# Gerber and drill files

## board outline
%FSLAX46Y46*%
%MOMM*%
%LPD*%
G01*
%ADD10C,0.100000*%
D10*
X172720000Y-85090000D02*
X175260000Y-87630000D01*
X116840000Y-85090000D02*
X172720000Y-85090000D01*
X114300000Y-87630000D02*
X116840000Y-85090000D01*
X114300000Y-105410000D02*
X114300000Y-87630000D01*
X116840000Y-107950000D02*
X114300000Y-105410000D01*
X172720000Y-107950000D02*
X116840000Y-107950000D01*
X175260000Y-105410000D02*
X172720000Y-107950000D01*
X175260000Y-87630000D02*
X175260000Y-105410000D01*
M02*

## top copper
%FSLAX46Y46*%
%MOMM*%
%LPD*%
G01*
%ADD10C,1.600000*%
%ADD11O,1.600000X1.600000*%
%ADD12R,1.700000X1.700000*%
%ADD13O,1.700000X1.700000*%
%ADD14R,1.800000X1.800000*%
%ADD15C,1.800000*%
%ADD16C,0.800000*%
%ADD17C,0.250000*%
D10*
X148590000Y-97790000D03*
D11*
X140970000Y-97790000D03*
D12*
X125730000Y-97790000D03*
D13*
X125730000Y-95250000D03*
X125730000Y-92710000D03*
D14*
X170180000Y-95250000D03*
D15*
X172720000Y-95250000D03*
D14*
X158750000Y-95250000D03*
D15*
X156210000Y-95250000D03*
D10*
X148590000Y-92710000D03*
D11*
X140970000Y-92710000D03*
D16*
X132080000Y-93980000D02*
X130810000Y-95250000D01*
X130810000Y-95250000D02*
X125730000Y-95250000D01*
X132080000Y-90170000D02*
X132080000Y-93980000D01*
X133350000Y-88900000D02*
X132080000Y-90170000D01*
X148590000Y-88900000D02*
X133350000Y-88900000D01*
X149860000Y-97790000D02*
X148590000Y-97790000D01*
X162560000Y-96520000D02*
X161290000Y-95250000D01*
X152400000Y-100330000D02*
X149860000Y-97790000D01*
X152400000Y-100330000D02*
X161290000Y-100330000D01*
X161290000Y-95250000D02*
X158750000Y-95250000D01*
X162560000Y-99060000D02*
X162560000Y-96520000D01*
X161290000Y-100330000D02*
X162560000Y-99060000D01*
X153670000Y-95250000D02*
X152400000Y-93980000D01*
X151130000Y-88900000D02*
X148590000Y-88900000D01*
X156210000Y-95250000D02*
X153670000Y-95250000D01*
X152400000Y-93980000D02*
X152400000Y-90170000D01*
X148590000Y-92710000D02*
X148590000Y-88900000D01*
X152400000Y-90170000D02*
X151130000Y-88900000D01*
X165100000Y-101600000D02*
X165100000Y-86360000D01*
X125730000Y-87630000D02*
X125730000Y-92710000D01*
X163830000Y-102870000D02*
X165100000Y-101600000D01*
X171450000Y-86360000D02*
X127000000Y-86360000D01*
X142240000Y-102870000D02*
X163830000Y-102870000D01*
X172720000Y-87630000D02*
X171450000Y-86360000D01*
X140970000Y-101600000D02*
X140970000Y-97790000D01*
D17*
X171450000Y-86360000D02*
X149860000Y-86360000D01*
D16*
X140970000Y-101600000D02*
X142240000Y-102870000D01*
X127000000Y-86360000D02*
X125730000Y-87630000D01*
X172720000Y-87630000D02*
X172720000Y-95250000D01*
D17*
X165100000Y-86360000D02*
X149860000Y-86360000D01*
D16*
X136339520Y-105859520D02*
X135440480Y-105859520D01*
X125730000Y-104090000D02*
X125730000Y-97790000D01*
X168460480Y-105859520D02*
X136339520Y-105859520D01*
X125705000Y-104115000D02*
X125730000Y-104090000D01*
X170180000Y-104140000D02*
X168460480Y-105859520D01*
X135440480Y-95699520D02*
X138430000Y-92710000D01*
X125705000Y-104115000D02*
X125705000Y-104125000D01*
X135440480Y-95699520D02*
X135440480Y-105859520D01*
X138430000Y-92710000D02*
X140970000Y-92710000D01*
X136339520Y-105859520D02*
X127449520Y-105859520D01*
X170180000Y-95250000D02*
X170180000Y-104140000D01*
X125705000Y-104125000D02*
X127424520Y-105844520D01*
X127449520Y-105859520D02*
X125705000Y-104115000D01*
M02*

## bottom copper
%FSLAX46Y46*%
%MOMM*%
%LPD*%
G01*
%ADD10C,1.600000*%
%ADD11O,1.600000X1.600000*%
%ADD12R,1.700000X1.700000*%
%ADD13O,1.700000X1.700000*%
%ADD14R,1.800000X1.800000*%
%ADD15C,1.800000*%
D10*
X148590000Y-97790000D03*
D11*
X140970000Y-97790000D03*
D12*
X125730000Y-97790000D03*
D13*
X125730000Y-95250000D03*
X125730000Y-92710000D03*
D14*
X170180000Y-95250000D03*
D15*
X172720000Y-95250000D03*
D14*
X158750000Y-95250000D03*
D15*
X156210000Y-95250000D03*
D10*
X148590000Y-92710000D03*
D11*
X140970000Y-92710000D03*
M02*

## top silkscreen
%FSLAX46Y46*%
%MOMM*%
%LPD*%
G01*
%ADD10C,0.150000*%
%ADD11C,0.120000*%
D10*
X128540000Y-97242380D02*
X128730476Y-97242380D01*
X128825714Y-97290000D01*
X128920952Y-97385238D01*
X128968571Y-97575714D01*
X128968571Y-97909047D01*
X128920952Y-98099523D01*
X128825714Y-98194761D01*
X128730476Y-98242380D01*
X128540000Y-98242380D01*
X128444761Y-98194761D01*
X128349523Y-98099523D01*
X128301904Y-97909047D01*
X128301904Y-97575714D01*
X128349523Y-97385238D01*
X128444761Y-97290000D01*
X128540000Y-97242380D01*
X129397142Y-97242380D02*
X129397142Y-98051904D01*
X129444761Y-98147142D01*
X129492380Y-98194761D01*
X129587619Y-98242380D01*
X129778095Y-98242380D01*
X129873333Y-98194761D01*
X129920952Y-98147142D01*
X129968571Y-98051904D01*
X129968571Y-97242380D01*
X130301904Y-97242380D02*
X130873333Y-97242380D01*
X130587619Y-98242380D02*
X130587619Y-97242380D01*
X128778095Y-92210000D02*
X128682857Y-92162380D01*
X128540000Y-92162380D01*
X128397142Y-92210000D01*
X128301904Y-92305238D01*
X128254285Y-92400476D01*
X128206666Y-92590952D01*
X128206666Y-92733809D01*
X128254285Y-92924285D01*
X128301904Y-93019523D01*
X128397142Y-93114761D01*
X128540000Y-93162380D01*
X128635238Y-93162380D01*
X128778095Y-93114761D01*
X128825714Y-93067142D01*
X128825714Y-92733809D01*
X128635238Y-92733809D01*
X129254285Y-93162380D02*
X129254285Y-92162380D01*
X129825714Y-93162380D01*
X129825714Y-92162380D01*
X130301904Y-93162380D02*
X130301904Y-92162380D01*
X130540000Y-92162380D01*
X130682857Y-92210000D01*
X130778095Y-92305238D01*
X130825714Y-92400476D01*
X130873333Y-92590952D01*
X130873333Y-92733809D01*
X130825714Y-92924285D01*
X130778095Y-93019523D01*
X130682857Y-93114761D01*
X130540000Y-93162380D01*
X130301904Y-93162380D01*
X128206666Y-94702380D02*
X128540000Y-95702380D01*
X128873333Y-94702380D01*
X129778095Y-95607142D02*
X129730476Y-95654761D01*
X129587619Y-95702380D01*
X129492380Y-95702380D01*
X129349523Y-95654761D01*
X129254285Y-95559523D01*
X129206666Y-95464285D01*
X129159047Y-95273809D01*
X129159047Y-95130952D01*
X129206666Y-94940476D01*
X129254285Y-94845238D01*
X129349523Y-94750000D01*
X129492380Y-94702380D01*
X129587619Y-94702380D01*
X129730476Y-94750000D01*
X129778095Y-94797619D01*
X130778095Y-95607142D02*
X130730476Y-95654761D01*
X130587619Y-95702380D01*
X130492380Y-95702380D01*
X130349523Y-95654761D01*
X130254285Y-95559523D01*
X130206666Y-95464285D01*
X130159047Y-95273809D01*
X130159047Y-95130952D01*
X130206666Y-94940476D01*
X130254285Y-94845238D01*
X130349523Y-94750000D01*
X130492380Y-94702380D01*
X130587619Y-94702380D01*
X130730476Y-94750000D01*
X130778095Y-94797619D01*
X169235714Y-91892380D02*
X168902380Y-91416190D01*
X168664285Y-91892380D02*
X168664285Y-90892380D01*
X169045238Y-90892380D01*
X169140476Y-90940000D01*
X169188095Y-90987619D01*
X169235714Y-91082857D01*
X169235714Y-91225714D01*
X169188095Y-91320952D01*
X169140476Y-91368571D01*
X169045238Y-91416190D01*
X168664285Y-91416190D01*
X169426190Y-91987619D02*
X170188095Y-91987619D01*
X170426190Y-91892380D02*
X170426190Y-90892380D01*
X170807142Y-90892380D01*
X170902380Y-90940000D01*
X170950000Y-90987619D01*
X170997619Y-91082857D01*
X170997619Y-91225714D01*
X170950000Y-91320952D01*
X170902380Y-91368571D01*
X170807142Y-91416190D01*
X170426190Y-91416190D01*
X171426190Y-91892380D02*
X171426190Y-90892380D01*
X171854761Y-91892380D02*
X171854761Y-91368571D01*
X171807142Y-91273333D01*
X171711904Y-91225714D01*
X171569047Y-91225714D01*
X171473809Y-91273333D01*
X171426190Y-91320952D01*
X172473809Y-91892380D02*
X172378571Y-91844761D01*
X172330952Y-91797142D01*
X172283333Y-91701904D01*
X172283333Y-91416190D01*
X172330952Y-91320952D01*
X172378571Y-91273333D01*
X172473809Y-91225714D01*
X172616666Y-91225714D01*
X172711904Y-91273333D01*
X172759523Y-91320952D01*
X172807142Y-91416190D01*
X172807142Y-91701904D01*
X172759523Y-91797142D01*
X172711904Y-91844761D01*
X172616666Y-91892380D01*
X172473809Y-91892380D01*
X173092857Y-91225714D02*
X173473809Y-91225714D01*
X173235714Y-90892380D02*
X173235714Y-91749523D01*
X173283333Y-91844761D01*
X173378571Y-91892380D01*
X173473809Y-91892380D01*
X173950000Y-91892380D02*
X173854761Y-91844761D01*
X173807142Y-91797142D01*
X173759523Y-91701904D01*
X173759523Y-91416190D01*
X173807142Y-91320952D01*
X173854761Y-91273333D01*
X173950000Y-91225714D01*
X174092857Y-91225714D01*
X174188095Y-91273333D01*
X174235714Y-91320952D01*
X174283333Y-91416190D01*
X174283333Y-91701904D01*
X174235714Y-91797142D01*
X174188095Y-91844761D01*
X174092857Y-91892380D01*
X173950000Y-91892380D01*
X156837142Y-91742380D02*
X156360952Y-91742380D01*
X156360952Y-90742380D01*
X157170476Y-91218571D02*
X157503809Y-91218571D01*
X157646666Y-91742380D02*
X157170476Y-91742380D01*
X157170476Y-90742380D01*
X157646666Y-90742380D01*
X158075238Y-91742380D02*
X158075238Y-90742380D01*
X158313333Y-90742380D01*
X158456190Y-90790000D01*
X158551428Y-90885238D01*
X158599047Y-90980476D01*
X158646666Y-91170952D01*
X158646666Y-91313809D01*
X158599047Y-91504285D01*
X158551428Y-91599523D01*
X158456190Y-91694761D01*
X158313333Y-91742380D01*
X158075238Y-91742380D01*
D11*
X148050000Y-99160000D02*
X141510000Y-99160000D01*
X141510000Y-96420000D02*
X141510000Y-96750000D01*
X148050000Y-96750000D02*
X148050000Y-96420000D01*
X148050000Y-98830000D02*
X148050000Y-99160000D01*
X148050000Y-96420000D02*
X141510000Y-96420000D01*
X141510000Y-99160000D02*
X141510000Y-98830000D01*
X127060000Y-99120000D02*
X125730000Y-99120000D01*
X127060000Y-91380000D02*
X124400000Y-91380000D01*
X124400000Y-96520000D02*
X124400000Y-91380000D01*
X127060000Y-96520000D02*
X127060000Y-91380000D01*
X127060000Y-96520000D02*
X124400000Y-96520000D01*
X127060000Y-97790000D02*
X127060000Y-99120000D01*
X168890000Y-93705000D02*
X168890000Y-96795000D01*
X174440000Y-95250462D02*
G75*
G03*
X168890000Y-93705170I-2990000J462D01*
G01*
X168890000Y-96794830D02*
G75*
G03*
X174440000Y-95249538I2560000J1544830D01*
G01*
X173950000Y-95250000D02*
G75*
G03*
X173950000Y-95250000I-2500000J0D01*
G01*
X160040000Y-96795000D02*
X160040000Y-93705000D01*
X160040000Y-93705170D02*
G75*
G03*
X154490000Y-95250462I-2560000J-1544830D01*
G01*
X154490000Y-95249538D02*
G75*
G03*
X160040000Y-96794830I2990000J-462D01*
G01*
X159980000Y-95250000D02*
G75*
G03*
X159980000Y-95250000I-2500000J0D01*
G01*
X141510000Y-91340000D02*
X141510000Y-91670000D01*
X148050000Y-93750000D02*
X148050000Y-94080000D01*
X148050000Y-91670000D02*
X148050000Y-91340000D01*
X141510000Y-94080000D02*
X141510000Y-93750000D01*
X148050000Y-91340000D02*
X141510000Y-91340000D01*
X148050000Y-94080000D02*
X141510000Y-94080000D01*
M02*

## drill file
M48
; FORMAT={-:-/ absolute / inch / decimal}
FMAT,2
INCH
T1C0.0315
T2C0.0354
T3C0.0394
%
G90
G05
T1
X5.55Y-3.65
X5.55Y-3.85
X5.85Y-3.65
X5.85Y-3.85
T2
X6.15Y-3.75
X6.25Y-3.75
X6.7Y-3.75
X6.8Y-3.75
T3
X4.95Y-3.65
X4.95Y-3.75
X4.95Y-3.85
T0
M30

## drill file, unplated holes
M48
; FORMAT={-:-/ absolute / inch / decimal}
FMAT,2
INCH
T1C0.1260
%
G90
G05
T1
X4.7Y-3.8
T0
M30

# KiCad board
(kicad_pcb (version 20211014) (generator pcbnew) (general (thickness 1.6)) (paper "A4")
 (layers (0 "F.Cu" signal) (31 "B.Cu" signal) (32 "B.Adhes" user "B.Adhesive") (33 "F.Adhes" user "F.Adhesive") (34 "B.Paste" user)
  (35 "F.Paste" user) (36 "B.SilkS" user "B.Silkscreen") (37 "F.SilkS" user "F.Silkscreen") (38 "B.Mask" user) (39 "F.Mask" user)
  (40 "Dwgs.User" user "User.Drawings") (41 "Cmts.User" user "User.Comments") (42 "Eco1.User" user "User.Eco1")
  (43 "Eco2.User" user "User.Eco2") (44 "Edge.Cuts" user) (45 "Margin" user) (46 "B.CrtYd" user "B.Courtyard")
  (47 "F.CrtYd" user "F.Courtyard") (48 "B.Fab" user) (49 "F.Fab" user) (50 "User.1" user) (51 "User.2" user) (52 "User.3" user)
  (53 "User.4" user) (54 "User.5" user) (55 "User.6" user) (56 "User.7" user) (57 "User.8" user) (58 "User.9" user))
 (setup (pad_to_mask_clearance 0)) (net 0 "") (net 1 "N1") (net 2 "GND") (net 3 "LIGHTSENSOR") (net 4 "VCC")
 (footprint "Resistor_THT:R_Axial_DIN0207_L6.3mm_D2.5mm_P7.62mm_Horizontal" (layer "F.Cu") (at 148.59 97.79 180)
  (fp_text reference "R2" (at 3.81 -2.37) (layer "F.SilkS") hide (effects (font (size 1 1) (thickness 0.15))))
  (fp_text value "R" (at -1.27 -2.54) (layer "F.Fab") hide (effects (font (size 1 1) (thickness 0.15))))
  (fp_line (start 0.54 -1.37) (end 7.08 -1.37) (layer "F.SilkS") (width 0.12))
  (fp_line (start 7.08 1.37) (end 7.08 1.04) (layer "F.SilkS") (width 0.12))
  (fp_line (start 0.54 1.04) (end 0.54 1.37) (layer "F.SilkS") (width 0.12))
  (fp_line (start 0.54 -1.04) (end 0.54 -1.37) (layer "F.SilkS") (width 0.12))
  (fp_line (start 0.54 1.37) (end 7.08 1.37) (layer "F.SilkS") (width 0.12))
  (fp_line (start 7.08 -1.37) (end 7.08 -1.04) (layer "F.SilkS") (width 0.12))
  (pad "1" thru_hole circle locked (at 0 0 180) (size 1.6 1.6) (drill 0.8) (layers *.Cu *.Mask) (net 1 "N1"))
  (pad "2" thru_hole oval locked (at 7.62 0 180) (size 1.6 1.6) (drill 0.8) (layers *.Cu *.Mask) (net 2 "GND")))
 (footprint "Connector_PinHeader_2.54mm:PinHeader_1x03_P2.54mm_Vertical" (layer "F.Cu") (at 125.73 97.79 180)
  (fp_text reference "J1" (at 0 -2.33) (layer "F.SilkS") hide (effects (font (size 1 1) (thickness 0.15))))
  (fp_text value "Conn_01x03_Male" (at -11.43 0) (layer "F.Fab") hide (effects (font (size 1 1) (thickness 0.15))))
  (fp_line (start -1.33 -1.33) (end 0 -1.33) (layer "F.SilkS") (width 0.12))
  (fp_line (start -1.33 6.41) (end 1.33 6.41) (layer "F.SilkS") (width 0.12))
  (fp_line (start 1.33 1.27) (end 1.33 6.41) (layer "F.SilkS") (width 0.12))
  (fp_line (start -1.33 1.27) (end -1.33 6.41) (layer "F.SilkS") (width 0.12))
  (fp_line (start -1.33 1.27) (end 1.33 1.27) (layer "F.SilkS") (width 0.12))
  (fp_line (start -1.33 0) (end -1.33 -1.33) (layer "F.SilkS") (width 0.12))
  (pad "1" thru_hole rect locked (at 0 0 180) (size 1.7 1.7) (drill 1) (layers *.Cu *.Mask) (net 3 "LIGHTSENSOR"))
  (pad "2" thru_hole oval locked (at 0 2.54 180) (size 1.7 1.7) (drill 1) (layers *.Cu *.Mask) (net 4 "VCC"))
  (pad "3" thru_hole oval locked (at 0 5.08 180) (size 1.7 1.7) (drill 1) (layers *.Cu *.Mask) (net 2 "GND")))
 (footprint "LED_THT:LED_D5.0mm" (layer "F.Cu") (at 170.18 95.25)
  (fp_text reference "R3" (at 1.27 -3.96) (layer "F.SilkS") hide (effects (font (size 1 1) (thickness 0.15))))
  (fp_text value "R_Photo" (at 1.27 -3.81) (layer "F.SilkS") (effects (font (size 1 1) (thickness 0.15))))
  (fp_line (start -1.29 -1.545) (end -1.29 1.545) (layer "F.SilkS") (width 0.12))
  (fp_arc (start -1.29 -1.54483) (mid 2.072002 -2.880433) (end 4.26 0.000462) (layer "F.SilkS") (width 0.12))
  (fp_arc (start 4.26 -0.000462) (mid 2.072002 2.880433) (end -1.29 1.54483) (layer "F.SilkS") (width 0.12))
  (fp_circle (center 1.27 0) (end 3.77 0) (layer "F.SilkS") (width 0.12) (fill none))
  (pad "1" thru_hole rect locked (at 0 0) (size 1.8 1.8) (drill 0.9) (layers *.Cu *.Mask) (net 3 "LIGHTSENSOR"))
  (pad "2" thru_hole circle locked (at 2.54 0) (size 1.8 1.8) (drill 0.9) (layers *.Cu *.Mask) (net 2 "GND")))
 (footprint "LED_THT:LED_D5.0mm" (layer "F.Cu") (at 158.75 95.25 180)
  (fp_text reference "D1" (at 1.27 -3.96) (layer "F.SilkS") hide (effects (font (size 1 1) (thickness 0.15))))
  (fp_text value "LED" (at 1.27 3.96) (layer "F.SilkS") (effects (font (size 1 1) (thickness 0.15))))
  (fp_line (start -1.29 -1.545) (end -1.29 1.545) (layer "F.SilkS") (width 0.12))
  (fp_arc (start 4.26 -0.000462) (mid 2.072002 2.880433) (end -1.29 1.54483) (layer "F.SilkS") (width 0.12))
  (fp_arc (start -1.29 -1.54483) (mid 2.072002 -2.880433) (end 4.26 0.000462) (layer "F.SilkS") (width 0.12))
  (fp_circle (center 1.27 0) (end 3.77 0) (layer "F.SilkS") (width 0.12) (fill none))
  (pad "1" thru_hole rect locked (at 0 0 180) (size 1.8 1.8) (drill 0.9) (layers *.Cu *.Mask) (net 1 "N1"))
  (pad "2" thru_hole circle locked (at 2.54 0 180) (size 1.8 1.8) (drill 0.9) (layers *.Cu *.Mask) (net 4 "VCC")))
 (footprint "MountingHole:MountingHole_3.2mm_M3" (layer "F.Cu") (at 119.38 96.52)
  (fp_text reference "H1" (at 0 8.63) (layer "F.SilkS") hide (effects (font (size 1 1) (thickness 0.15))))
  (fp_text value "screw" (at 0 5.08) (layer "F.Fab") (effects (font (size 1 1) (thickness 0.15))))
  (pad "" np_thru_hole circle locked (at 0 0) (size 3.2 3.2) (drill 3.2) (layers *.Cu *.Mask)))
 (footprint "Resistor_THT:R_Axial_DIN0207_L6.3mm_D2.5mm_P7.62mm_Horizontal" (layer "F.Cu") (at 148.59 92.71 180)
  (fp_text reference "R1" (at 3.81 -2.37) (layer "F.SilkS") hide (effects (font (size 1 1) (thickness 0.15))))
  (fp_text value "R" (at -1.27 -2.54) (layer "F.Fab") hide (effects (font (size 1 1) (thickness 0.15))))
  (fp_line (start 7.08 1.37) (end 7.08 1.04) (layer "F.SilkS") (width 0.12))
  (fp_line (start 0.54 -1.04) (end 0.54 -1.37) (layer "F.SilkS") (width 0.12))
  (fp_line (start 0.54 1.04) (end 0.54 1.37) (layer "F.SilkS") (width 0.12))
  (fp_line (start 7.08 -1.37) (end 7.08 -1.04) (layer "F.SilkS") (width 0.12))
  (fp_line (start 0.54 1.37) (end 7.08 1.37) (layer "F.SilkS") (width 0.12))
  (fp_line (start 0.54 -1.37) (end 7.08 -1.37) (layer "F.SilkS") (width 0.12))
  (pad "1" thru_hole circle locked (at 0 0 180) (size 1.6 1.6) (drill 0.8) (layers *.Cu *.Mask) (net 4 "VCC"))
  (pad "2" thru_hole oval locked (at 7.62 0 180) (size 1.6 1.6) (drill 0.8) (layers *.Cu *.Mask) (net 3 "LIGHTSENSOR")))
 (gr_line (start 114.3 105.41) (end 114.3 87.63) (layer "Edge.Cuts") (width 0.1))
 (gr_line (start 172.72 107.95) (end 116.84 107.95) (layer "Edge.Cuts") (width 0.1))
 (gr_line (start 116.84 107.95) (end 114.3 105.41) (layer "Edge.Cuts") (width 0.1))
 (gr_line (start 116.84 85.09) (end 172.72 85.09) (layer "Edge.Cuts") (width 0.1))
 (gr_line (start 172.72 85.09) (end 175.26 87.63) (layer "Edge.Cuts") (width 0.1))
 (gr_line (start 175.26 105.41) (end 172.72 107.95) (layer "Edge.Cuts") (width 0.1))
 (gr_line (start 175.26 87.63) (end 175.26 105.41) (layer "Edge.Cuts") (width 0.1))
 (gr_line (start 114.3 87.63) (end 116.84 85.09) (layer "Edge.Cuts") (width 0.1))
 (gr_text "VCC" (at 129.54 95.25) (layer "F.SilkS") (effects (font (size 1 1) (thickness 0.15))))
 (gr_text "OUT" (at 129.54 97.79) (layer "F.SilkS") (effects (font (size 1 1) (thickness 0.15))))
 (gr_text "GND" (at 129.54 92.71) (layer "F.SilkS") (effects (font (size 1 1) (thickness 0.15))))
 (segment (start 149.86 97.79) (end 148.59 97.79) (width 0.8) (layer "F.Cu") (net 1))
 (segment (start 162.56 96.52) (end 161.29 95.25) (width 0.8) (layer "F.Cu") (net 1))
 (segment (start 152.4 100.33) (end 149.86 97.79) (width 0.8) (layer "F.Cu") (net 1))
 (segment (start 152.4 100.33) (end 161.29 100.33) (width 0.8) (layer "F.Cu") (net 1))
 (segment (start 161.29 95.25) (end 158.75 95.25) (width 0.8) (layer "F.Cu") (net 1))
 (segment (start 162.56 99.06) (end 162.56 96.52) (width 0.8) (layer "F.Cu") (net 1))
 (segment (start 161.29 100.33) (end 162.56 99.06) (width 0.8) (layer "F.Cu") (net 1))
 (segment (start 153.67 95.25) (end 152.4 93.98) (width 0.8) (layer "F.Cu") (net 4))
 (segment (start 132.08 90.17) (end 132.08 93.98) (width 0.8) (layer "F.Cu") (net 4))
 (segment (start 151.13 88.9) (end 148.59 88.9) (width 0.8) (layer "F.Cu") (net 4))
 (segment (start 156.21 95.25) (end 153.67 95.25) (width 0.8) (layer "F.Cu") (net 4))
 (segment (start 130.81 95.25) (end 125.73 95.25) (width 0.8) (layer "F.Cu") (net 4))
 (segment (start 152.4 93.98) (end 152.4 90.17) (width 0.8) (layer "F.Cu") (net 4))
 (segment (start 133.35 88.9) (end 132.08 90.17) (width 0.8) (layer "F.Cu") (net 4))
 (segment (start 148.59 88.9) (end 133.35 88.9) (width 0.8) (layer "F.Cu") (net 4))
 (segment (start 148.59 92.71) (end 148.59 88.9) (width 0.8) (layer "F.Cu") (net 4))
 (segment (start 132.08 93.98) (end 130.81 95.25) (width 0.8) (layer "F.Cu") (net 4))
 (segment (start 152.4 90.17) (end 151.13 88.9) (width 0.8) (layer "F.Cu") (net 4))
 (segment (start 165.1 101.6) (end 165.1 86.36) (width 0.8) (layer "F.Cu") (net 2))
 (segment (start 125.73 87.63) (end 125.73 92.71) (width 0.8) (layer "F.Cu") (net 2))
 (segment (start 163.83 102.87) (end 165.1 101.6) (width 0.8) (layer "F.Cu") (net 2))
 (segment (start 171.45 86.36) (end 127 86.36) (width 0.8) (layer "F.Cu") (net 2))
 (segment (start 142.24 102.87) (end 163.83 102.87) (width 0.8) (layer "F.Cu") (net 2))
 (segment (start 172.72 87.63) (end 171.45 86.36) (width 0.8) (layer "F.Cu") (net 2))
 (segment (start 140.97 101.6) (end 140.97 97.79) (width 0.8) (layer "F.Cu") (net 2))
 (segment (start 171.45 86.36) (end 149.86 86.36) (width 0.25) (layer "F.Cu") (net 2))
 (segment (start 140.97 101.6) (end 142.24 102.87) (width 0.8) (layer "F.Cu") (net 2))
 (segment (start 127 86.36) (end 125.73 87.63) (width 0.8) (layer "F.Cu") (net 2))
 (segment (start 172.72 87.63) (end 172.72 95.25) (width 0.8) (layer "F.Cu") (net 2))
 (segment (start 165.1 86.36) (end 149.86 86.36) (width 0.25) (layer "F.Cu") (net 2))
 (segment (start 136.33952 105.85952) (end 135.44048 105.85952) (width 0.8) (layer "F.Cu") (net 3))
 (segment (start 125.73 104.09) (end 125.73 97.79) (width 0.8) (layer "F.Cu") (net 3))
 (segment (start 168.46048 105.85952) (end 136.33952 105.85952) (width 0.8) (layer "F.Cu") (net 3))
 (segment (start 125.705 104.115) (end 125.73 104.09) (width 0.8) (layer "F.Cu") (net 3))
 (segment (start 170.18 104.14) (end 168.46048 105.85952) (width 0.8) (layer "F.Cu") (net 3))
 (segment (start 135.44048 95.69952) (end 138.43 92.71) (width 0.8) (layer "F.Cu") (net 3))
 (segment (start 125.705 104.115) (end 125.705 104.125) (width 0.8) (layer "F.Cu") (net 3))
 (segment (start 135.44048 95.69952) (end 135.44048 105.85952) (width 0.8) (layer "F.Cu") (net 3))
 (segment (start 138.43 92.71) (end 140.97 92.71) (width 0.8) (layer "F.Cu") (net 3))
 (segment (start 136.33952 105.85952) (end 127.44952 105.85952) (width 0.8) (layer "F.Cu") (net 3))
 (segment (start 170.18 95.25) (end 170.18 104.14) (width 0.8) (layer "F.Cu") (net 3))
 (segment (start 125.705 104.125) (end 127.42452 105.84452) (width 0.8) (layer "F.Cu") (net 3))
 (segment (start 127.44952 105.85952) (end 125.705 104.115) (width 0.8) (layer "F.Cu") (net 3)))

